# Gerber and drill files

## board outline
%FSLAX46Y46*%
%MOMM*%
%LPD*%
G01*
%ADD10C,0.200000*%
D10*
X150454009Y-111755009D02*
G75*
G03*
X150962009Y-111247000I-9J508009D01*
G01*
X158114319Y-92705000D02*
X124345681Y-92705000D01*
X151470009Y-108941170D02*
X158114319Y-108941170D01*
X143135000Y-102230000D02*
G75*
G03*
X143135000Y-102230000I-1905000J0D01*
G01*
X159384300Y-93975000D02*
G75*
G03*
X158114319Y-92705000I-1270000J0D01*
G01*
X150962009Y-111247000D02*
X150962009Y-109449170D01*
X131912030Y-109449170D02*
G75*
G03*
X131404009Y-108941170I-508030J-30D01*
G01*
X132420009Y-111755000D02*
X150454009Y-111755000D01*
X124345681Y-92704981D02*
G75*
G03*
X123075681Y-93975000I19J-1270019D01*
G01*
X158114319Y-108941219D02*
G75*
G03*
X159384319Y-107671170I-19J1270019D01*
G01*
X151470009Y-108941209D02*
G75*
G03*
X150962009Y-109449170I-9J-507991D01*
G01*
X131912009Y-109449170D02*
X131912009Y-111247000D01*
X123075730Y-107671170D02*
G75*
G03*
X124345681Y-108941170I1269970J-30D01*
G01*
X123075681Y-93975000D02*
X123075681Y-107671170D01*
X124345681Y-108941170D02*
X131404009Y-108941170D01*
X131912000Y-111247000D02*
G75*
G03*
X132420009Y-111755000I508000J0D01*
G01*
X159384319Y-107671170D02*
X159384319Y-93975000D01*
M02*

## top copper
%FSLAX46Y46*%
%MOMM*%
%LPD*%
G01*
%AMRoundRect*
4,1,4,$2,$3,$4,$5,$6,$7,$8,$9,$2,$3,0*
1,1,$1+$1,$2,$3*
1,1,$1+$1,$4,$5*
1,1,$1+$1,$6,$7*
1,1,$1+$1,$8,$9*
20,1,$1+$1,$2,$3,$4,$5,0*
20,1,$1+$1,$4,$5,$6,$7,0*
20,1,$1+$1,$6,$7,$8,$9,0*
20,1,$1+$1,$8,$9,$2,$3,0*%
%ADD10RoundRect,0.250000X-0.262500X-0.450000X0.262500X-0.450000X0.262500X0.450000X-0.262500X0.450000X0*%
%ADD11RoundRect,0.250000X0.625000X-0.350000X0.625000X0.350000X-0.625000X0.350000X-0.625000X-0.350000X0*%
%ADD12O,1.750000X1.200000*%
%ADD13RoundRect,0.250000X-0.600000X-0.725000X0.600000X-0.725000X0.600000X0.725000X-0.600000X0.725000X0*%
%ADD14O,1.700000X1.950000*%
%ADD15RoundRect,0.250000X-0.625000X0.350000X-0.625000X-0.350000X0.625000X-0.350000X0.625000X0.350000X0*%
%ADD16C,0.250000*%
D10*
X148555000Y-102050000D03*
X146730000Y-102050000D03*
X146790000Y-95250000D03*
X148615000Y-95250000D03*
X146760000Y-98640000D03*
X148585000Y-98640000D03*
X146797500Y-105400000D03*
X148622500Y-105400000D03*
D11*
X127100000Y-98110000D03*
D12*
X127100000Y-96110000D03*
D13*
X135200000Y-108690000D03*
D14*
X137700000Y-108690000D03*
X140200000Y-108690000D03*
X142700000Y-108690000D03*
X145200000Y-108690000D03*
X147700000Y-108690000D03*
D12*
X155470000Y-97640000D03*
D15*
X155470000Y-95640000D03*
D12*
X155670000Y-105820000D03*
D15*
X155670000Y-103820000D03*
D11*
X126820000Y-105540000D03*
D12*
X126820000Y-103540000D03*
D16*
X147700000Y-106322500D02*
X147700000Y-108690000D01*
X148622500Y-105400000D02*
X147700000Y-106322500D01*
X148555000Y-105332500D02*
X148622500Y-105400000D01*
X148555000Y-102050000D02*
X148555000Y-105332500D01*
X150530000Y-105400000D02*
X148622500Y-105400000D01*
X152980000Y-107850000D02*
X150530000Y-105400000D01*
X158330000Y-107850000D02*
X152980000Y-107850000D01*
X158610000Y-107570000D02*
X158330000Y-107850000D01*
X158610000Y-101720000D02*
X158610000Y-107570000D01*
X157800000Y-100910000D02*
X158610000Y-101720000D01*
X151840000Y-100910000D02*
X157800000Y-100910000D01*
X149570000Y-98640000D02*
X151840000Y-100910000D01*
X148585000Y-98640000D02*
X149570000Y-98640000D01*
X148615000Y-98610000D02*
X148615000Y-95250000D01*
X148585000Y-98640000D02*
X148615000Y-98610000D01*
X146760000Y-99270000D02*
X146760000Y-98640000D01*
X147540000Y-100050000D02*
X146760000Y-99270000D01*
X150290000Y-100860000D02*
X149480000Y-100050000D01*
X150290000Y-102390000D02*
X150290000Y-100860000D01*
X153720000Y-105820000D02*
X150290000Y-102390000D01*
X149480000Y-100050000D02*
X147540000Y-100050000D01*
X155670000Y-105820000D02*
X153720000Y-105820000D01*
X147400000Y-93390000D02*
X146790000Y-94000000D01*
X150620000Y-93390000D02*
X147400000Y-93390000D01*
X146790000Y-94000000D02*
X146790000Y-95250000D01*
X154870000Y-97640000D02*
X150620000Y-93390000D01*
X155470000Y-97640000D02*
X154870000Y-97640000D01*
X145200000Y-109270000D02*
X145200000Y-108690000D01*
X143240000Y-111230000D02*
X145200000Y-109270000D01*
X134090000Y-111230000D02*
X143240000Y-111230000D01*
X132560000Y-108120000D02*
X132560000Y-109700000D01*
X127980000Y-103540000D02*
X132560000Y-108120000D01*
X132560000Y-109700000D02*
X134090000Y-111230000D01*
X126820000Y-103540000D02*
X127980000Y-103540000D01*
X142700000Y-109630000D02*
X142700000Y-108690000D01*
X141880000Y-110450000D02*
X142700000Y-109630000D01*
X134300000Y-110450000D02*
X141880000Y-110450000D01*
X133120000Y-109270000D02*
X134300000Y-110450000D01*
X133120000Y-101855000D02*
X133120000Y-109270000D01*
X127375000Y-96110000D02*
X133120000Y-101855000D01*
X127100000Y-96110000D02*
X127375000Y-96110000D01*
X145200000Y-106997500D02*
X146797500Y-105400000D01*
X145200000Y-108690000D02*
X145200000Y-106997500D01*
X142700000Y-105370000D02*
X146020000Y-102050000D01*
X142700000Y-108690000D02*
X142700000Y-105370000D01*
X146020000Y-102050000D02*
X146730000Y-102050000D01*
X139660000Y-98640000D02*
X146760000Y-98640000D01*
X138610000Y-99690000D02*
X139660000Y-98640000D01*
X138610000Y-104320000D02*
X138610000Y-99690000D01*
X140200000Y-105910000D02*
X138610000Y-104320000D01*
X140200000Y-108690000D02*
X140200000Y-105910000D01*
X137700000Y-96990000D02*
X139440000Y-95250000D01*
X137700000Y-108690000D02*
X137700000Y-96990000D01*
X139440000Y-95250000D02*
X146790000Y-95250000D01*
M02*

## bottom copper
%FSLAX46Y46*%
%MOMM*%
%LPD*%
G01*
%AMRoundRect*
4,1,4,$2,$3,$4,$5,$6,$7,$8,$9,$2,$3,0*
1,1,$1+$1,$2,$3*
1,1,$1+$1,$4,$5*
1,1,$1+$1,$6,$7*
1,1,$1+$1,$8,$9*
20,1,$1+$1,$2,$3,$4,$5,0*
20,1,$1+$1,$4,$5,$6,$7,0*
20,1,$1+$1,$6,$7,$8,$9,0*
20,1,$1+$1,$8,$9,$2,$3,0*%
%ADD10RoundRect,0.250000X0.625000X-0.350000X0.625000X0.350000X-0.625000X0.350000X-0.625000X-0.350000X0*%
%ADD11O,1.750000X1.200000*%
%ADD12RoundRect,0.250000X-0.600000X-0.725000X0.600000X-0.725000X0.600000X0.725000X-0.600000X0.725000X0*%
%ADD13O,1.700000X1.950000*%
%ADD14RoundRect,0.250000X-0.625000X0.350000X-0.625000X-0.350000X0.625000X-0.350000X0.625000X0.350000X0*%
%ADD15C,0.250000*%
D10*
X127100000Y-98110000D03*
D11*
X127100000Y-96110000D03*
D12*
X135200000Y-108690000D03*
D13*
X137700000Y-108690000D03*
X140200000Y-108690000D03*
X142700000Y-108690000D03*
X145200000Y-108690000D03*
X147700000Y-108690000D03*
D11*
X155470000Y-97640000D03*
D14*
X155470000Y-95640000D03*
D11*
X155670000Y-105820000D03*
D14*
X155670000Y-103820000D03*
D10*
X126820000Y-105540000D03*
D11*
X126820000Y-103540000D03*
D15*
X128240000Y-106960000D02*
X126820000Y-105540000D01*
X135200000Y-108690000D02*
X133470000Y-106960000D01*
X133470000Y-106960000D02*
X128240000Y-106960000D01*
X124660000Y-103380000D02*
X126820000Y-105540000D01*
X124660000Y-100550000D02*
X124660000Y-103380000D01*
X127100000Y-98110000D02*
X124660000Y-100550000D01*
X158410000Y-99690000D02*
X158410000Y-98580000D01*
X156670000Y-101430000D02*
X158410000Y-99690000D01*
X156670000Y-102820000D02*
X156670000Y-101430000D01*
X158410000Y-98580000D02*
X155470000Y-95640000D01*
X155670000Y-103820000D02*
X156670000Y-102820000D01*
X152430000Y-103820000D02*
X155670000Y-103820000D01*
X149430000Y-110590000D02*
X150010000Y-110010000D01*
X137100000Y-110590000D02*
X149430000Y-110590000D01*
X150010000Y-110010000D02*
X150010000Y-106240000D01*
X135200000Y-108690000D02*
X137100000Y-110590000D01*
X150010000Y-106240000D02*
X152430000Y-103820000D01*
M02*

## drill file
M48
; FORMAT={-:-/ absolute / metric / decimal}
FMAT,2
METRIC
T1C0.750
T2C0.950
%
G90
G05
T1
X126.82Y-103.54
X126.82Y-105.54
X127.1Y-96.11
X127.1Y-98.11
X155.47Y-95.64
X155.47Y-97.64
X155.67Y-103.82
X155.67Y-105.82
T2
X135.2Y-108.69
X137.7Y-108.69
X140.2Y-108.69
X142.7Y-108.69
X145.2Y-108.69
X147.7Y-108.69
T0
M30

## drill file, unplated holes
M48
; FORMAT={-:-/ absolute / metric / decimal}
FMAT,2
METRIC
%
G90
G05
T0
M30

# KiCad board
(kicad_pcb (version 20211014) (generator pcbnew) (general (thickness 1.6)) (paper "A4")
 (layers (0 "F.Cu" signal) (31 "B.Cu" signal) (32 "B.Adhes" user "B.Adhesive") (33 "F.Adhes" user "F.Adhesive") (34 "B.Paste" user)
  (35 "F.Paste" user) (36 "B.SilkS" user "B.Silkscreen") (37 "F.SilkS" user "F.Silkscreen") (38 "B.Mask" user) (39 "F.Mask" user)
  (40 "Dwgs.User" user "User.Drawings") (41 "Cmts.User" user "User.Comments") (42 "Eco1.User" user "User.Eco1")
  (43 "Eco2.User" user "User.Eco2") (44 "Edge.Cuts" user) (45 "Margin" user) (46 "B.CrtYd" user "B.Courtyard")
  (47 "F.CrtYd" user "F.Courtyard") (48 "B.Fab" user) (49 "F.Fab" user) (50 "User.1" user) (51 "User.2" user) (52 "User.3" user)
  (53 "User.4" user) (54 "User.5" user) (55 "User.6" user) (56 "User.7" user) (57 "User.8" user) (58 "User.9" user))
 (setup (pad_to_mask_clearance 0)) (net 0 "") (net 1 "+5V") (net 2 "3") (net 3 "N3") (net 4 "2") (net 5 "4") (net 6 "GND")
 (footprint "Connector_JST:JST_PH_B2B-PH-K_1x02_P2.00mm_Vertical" (layer "F.Cu") (at 127.1 98.11 90)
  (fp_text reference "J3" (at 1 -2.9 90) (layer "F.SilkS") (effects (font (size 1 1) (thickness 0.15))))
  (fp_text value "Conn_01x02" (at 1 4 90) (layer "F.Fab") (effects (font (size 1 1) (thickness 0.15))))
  (pad "1" thru_hole roundrect (at 0 0 90) (size 1.2 1.75) (drill 0.75) (layers *.Cu *.Mask) (roundrect_rratio 0.2083333333) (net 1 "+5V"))
  (pad "2" thru_hole oval (at 2 0 90) (size 1.2 1.75) (drill 0.75) (layers *.Cu *.Mask) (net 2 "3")))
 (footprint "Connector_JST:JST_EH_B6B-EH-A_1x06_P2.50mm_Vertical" (layer "F.Cu") (at 135.2 108.69)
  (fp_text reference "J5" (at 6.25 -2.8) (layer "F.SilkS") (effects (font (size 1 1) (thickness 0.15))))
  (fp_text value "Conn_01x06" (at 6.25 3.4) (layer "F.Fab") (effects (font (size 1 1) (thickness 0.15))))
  (pad "1" thru_hole roundrect (at 0 0) (size 1.7 1.95) (drill 0.95) (layers *.Cu *.Mask) (roundrect_rratio 0.1470588235) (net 1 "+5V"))
  (pad "2" thru_hole oval (at 2.5 0) (size 1.7 1.95) (drill 0.95) (layers *.Cu *.Mask) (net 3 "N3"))
  (pad "3" thru_hole oval (at 5 0) (size 1.7 1.95) (drill 0.95) (layers *.Cu *.Mask) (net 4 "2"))
  (pad "4" thru_hole oval (at 7.5 0) (size 1.7 1.95) (drill 0.95) (layers *.Cu *.Mask) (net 2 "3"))
  (pad "5" thru_hole oval (at 10 0) (size 1.7 1.95) (drill 0.95) (layers *.Cu *.Mask) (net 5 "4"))
  (pad "6" thru_hole oval (at 12.5 0) (size 1.7 1.95) (drill 0.95) (layers *.Cu *.Mask) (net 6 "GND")))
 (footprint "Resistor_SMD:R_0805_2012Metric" (layer "F.Cu") (at 147.71 105.4)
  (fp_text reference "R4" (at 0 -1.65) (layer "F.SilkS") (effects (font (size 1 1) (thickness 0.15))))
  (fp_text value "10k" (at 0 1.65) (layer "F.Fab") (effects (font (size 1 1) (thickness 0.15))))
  (pad "1" smd roundrect (at -0.9125 0) (size 1.025 1.4) (layers "F.Cu" "F.Paste" "F.Mask") (roundrect_rratio 0.243902439) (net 5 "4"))
  (pad "2" smd roundrect (at 0.9125 0) (size 1.025 1.4) (layers "F.Cu" "F.Paste" "F.Mask") (roundrect_rratio 0.243902439) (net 6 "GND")))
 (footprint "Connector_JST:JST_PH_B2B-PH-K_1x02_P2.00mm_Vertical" (layer "F.Cu") (at 155.47 95.64 -90)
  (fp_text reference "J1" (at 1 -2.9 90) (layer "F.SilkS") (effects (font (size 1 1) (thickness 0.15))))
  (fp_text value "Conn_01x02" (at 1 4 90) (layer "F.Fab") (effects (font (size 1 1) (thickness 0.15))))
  (pad "1" thru_hole roundrect (at 0 0 270) (size 1.2 1.75) (drill 0.75) (layers *.Cu *.Mask) (roundrect_rratio 0.2083333333) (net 1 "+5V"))
  (pad "2" thru_hole oval (at 2 0 270) (size 1.2 1.75) (drill 0.75) (layers *.Cu *.Mask) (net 3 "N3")))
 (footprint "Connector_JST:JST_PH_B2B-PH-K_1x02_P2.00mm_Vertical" (layer "F.Cu") (at 155.67 103.82 -90)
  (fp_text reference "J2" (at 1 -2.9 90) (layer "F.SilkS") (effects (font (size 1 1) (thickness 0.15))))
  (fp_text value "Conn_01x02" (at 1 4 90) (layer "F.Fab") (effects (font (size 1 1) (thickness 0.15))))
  (pad "1" thru_hole roundrect (at 0 0 270) (size 1.2 1.75) (drill 0.75) (layers *.Cu *.Mask) (roundrect_rratio 0.2083333333) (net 1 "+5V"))
  (pad "2" thru_hole oval (at 2 0 270) (size 1.2 1.75) (drill 0.75) (layers *.Cu *.Mask) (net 4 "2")))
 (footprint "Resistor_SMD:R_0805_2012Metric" (layer "F.Cu") (at 147.6725 98.64)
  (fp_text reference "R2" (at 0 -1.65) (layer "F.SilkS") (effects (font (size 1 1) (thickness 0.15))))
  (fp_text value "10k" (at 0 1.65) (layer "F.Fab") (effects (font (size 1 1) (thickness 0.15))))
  (pad "1" smd roundrect (at -0.9125 0) (size 1.025 1.4) (layers "F.Cu" "F.Paste" "F.Mask") (roundrect_rratio 0.243902439) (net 4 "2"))
  (pad "2" smd roundrect (at 0.9125 0) (size 1.025 1.4) (layers "F.Cu" "F.Paste" "F.Mask") (roundrect_rratio 0.243902439) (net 6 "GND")))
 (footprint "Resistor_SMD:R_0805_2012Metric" (layer "F.Cu") (at 147.6425 102.05)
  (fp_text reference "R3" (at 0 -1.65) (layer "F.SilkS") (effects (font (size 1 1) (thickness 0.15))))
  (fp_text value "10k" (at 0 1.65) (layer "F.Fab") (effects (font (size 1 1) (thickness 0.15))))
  (pad "1" smd roundrect (at -0.9125 0) (size 1.025 1.4) (layers "F.Cu" "F.Paste" "F.Mask") (roundrect_rratio 0.243902439) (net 2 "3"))
  (pad "2" smd roundrect (at 0.9125 0) (size 1.025 1.4) (layers "F.Cu" "F.Paste" "F.Mask") (roundrect_rratio 0.243902439) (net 6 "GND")))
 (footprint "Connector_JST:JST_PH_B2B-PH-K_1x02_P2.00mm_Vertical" (layer "F.Cu") (at 126.82 105.54 90)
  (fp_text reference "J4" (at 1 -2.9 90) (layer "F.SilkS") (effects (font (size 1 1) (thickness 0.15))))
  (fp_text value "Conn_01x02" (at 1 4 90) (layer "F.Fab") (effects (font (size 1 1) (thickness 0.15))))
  (pad "1" thru_hole roundrect (at 0 0 90) (size 1.2 1.75) (drill 0.75) (layers *.Cu *.Mask) (roundrect_rratio 0.2083333333) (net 1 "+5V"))
  (pad "2" thru_hole oval (at 2 0 90) (size 1.2 1.75) (drill 0.75) (layers *.Cu *.Mask) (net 5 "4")))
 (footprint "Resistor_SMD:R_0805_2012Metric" (layer "F.Cu") (at 147.7025 95.25)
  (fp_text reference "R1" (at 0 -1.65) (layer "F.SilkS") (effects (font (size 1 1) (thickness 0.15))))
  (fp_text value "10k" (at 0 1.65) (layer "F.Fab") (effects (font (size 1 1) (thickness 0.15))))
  (pad "1" smd roundrect (at -0.9125 0) (size 1.025 1.4) (layers "F.Cu" "F.Paste" "F.Mask") (roundrect_rratio 0.243902439) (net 3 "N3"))
  (pad "2" smd roundrect (at 0.9125 0) (size 1.025 1.4) (layers "F.Cu" "F.Paste" "F.Mask") (roundrect_rratio 0.243902439) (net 6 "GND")))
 (gr_arc (start 150.962009 111.247) (mid 150.81322 111.606211) (end 150.454009 111.755) (layer "Edge.Cuts") (width 0.2))
 (gr_line (start 158.114319 92.705) (end 124.345681 92.705) (layer "Edge.Cuts") (width 0.2))
 (gr_line (start 151.470009 108.94117) (end 158.114319 108.94117) (layer "Edge.Cuts") (width 0.2))
 (gr_circle (center 141.23 102.23) (end 143.135 102.23) (layer "Edge.Cuts") (width 0.2) (fill none))
 (gr_arc (start 158.114319 92.705) (mid 159.012345 93.076974) (end 159.384319 93.975) (layer "Edge.Cuts") (width 0.2))
 (gr_line (start 150.962009 111.247) (end 150.962009 109.44917) (layer "Edge.Cuts") (width 0.2))
 (gr_arc (start 131.404009 108.94117) (mid 131.76322 109.089959) (end 131.912009 109.44917) (layer "Edge.Cuts") (width 0.2))
 (gr_line (start 132.420009 111.755) (end 150.454009 111.755) (layer "Edge.Cuts") (width 0.2))
 (gr_arc (start 123.075681 93.975) (mid 123.447655 93.076974) (end 124.345681 92.705) (layer "Edge.Cuts") (width 0.2))
 (gr_arc (start 159.384319 107.67117) (mid 159.012345 108.569196) (end 158.114319 108.94117) (layer "Edge.Cuts") (width 0.2))
 (gr_arc (start 150.962009 109.44917) (mid 151.110798 109.089959) (end 151.470009 108.94117) (layer "Edge.Cuts") (width 0.2))
 (gr_line (start 131.912009 109.44917) (end 131.912009 111.247) (layer "Edge.Cuts") (width 0.2))
 (gr_arc (start 124.345681 108.94117) (mid 123.447655 108.569196) (end 123.075681 107.67117) (layer "Edge.Cuts") (width 0.2))
 (gr_line (start 123.075681 93.975) (end 123.075681 107.67117) (layer "Edge.Cuts") (width 0.2))
 (gr_line (start 124.345681 108.94117) (end 131.404009 108.94117) (layer "Edge.Cuts") (width 0.2))
 (gr_arc (start 132.420009 111.755) (mid 132.060799 111.60621) (end 131.912009 111.247) (layer "Edge.Cuts") (width 0.2))
 (gr_line (start 159.384319 107.67117) (end 159.384319 93.975) (layer "Edge.Cuts") (width 0.2))
 (segment (start 124.66 103.38) (end 126.82 105.54) (width 0.25) (layer "B.Cu") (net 1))
 (segment (start 150.01 110.01) (end 150.01 106.24) (width 0.25) (layer "B.Cu") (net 1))
 (segment (start 128.24 106.96) (end 126.82 105.54) (width 0.25) (layer "B.Cu") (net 1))
 (segment (start 135.2 108.69) (end 133.47 106.96) (width 0.25) (layer "B.Cu") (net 1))
 (segment (start 152.43 103.82) (end 155.67 103.82) (width 0.25) (layer "B.Cu") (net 1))
 (segment (start 124.66 100.55) (end 124.66 103.38) (width 0.25) (layer "B.Cu") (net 1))
 (segment (start 135.2 108.69) (end 137.1 110.59) (width 0.25) (layer "B.Cu") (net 1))
 (segment (start 133.47 106.96) (end 128.24 106.96) (width 0.25) (layer "B.Cu") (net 1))
 (segment (start 158.41 99.69) (end 158.41 98.58) (width 0.25) (layer "B.Cu") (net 1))
 (segment (start 158.41 98.58) (end 155.47 95.64) (width 0.25) (layer "B.Cu") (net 1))
 (segment (start 137.1 110.59) (end 149.43 110.59) (width 0.25) (layer "B.Cu") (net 1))
 (segment (start 156.67 102.82) (end 156.67 101.43) (width 0.25) (layer "B.Cu") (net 1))
 (segment (start 150.01 106.24) (end 152.43 103.82) (width 0.25) (layer "B.Cu") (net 1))
 (segment (start 149.43 110.59) (end 150.01 110.01) (width 0.25) (layer "B.Cu") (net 1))
 (segment (start 156.67 101.43) (end 158.41 99.69) (width 0.25) (layer "B.Cu") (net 1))
 (segment (start 155.67 103.82) (end 156.67 102.82) (width 0.25) (layer "B.Cu") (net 1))
 (segment (start 127.1 98.11) (end 124.66 100.55) (width 0.25) (layer "B.Cu") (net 1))
 (segment (start 155.47 97.64) (end 154.87 97.64) (width 0.25) (layer "F.Cu") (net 3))
 (segment (start 147.4 93.39) (end 146.79 94) (width 0.25) (layer "F.Cu") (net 3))
 (segment (start 137.7 96.99) (end 139.44 95.25) (width 0.25) (layer "F.Cu") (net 3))
 (segment (start 139.44 95.25) (end 146.79 95.25) (width 0.25) (layer "F.Cu") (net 3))
 (segment (start 137.7 108.69) (end 137.7 96.99) (width 0.25) (layer "F.Cu") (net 3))
 (segment (start 154.87 97.64) (end 150.62 93.39) (width 0.25) (layer "F.Cu") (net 3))
 (segment (start 146.79 94) (end 146.79 95.25) (width 0.25) (layer "F.Cu") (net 3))
 (segment (start 150.62 93.39) (end 147.4 93.39) (width 0.25) (layer "F.Cu") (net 3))
 (segment (start 149.48 100.05) (end 147.54 100.05) (width 0.25) (layer "F.Cu") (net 4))
 (segment (start 155.67 105.82) (end 153.72 105.82) (width 0.25) (layer "F.Cu") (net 4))
 (segment (start 140.2 108.69) (end 140.2 105.91) (width 0.25) (layer "F.Cu") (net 4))
 (segment (start 139.66 98.64) (end 146.76 98.64) (width 0.25) (layer "F.Cu") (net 4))
 (segment (start 150.29 100.86) (end 149.48 100.05) (width 0.25) (layer "F.Cu") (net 4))
 (segment (start 153.72 105.82) (end 150.29 102.39) (width 0.25) (layer "F.Cu") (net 4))
 (segment (start 147.54 100.05) (end 146.76 99.27) (width 0.25) (layer "F.Cu") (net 4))
 (segment (start 140.2 105.91) (end 138.61 104.32) (width 0.25) (layer "F.Cu") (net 4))
 (segment (start 138.61 99.69) (end 139.66 98.64) (width 0.25) (layer "F.Cu") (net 4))
 (segment (start 150.29 102.39) (end 150.29 100.86) (width 0.25) (layer "F.Cu") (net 4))
 (segment (start 138.61 104.32) (end 138.61 99.69) (width 0.25) (layer "F.Cu") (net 4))
 (segment (start 146.76 99.27) (end 146.76 98.64) (width 0.25) (layer "F.Cu") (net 4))
 (segment (start 142.7 108.69) (end 142.7 105.37) (width 0.25) (layer "F.Cu") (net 2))
 (segment (start 142.7 105.37) (end 146.02 102.05) (width 0.25) (layer "F.Cu") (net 2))
 (segment (start 142.7 109.63) (end 142.7 108.69) (width 0.25) (layer "F.Cu") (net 2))
 (segment (start 146.02 102.05) (end 146.73 102.05) (width 0.25) (layer "F.Cu") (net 2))
 (segment (start 127.1 96.11) (end 127.375 96.11) (width 0.25) (layer "F.Cu") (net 2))
 (segment (start 141.88 110.45) (end 142.7 109.63) (width 0.25) (layer "F.Cu") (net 2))
 (segment (start 133.12 109.27) (end 134.3 110.45) (width 0.25) (layer "F.Cu") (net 2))
 (segment (start 127.375 96.11) (end 133.12 101.855) (width 0.25) (layer "F.Cu") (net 2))
 (segment (start 134.3 110.45) (end 141.88 110.45) (width 0.25) (layer "F.Cu") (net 2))
 (segment (start 133.12 101.855) (end 133.12 109.27) (width 0.25) (layer "F.Cu") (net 2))
 (segment (start 145.2 108.69) (end 145.2 106.9975) (width 0.25) (layer "F.Cu") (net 5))
 (segment (start 126.82 103.54) (end 127.98 103.54) (width 0.25) (layer "F.Cu") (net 5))
 (segment (start 132.56 108.12) (end 132.56 109.7) (width 0.25) (layer "F.Cu") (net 5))
 (segment (start 134.09 111.23) (end 143.24 111.23) (width 0.25) (layer "F.Cu") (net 5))
 (segment (start 145.2 106.9975) (end 146.7975 105.4) (width 0.25) (layer "F.Cu") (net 5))
 (segment (start 143.24 111.23) (end 145.2 109.27) (width 0.25) (layer "F.Cu") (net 5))
 (segment (start 127.98 103.54) (end 132.56 108.12) (width 0.25) (layer "F.Cu") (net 5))
 (segment (start 145.2 109.27) (end 145.2 108.69) (width 0.25) (layer "F.Cu") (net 5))
 (segment (start 132.56 109.7) (end 134.09 111.23) (width 0.25) (layer "F.Cu") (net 5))
 (segment (start 158.61 101.72) (end 158.61 107.57) (width 0.25) (layer "F.Cu") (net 6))
 (segment (start 148.585 98.64) (end 148.615 98.61) (width 0.25) (layer "F.Cu") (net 6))
 (segment (start 148.555 102.05) (end 148.555 105.3325) (width 0.25) (layer "F.Cu") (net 6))
 (segment (start 157.8 100.91) (end 158.61 101.72) (width 0.25) (layer "F.Cu") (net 6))
 (segment (start 149.57 98.64) (end 151.84 100.91) (width 0.25) (layer "F.Cu") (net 6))
 (segment (start 158.61 107.57) (end 158.33 107.85) (width 0.25) (layer "F.Cu") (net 6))
 (segment (start 150.53 105.4) (end 148.6225 105.4) (width 0.25) (layer "F.Cu") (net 6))
 (segment (start 148.585 98.64) (end 149.57 98.64) (width 0.25) (layer "F.Cu") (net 6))
 (segment (start 148.6225 105.4) (end 147.7 106.3225) (width 0.25) (layer "F.Cu") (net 6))
 (segment (start 148.615 98.61) (end 148.615 95.25) (width 0.25) (layer "F.Cu") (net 6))
 (segment (start 148.555 105.3325) (end 148.6225 105.4) (width 0.25) (layer "F.Cu") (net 6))
 (segment (start 152.98 107.85) (end 150.53 105.4) (width 0.25) (layer "F.Cu") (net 6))
 (segment (start 147.7 106.3225) (end 147.7 108.69) (width 0.25) (layer "F.Cu") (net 6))
 (segment (start 158.33 107.85) (end 152.98 107.85) (width 0.25) (layer "F.Cu") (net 6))
 (segment (start 151.84 100.91) (end 157.8 100.91) (width 0.25) (layer "F.Cu") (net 6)))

